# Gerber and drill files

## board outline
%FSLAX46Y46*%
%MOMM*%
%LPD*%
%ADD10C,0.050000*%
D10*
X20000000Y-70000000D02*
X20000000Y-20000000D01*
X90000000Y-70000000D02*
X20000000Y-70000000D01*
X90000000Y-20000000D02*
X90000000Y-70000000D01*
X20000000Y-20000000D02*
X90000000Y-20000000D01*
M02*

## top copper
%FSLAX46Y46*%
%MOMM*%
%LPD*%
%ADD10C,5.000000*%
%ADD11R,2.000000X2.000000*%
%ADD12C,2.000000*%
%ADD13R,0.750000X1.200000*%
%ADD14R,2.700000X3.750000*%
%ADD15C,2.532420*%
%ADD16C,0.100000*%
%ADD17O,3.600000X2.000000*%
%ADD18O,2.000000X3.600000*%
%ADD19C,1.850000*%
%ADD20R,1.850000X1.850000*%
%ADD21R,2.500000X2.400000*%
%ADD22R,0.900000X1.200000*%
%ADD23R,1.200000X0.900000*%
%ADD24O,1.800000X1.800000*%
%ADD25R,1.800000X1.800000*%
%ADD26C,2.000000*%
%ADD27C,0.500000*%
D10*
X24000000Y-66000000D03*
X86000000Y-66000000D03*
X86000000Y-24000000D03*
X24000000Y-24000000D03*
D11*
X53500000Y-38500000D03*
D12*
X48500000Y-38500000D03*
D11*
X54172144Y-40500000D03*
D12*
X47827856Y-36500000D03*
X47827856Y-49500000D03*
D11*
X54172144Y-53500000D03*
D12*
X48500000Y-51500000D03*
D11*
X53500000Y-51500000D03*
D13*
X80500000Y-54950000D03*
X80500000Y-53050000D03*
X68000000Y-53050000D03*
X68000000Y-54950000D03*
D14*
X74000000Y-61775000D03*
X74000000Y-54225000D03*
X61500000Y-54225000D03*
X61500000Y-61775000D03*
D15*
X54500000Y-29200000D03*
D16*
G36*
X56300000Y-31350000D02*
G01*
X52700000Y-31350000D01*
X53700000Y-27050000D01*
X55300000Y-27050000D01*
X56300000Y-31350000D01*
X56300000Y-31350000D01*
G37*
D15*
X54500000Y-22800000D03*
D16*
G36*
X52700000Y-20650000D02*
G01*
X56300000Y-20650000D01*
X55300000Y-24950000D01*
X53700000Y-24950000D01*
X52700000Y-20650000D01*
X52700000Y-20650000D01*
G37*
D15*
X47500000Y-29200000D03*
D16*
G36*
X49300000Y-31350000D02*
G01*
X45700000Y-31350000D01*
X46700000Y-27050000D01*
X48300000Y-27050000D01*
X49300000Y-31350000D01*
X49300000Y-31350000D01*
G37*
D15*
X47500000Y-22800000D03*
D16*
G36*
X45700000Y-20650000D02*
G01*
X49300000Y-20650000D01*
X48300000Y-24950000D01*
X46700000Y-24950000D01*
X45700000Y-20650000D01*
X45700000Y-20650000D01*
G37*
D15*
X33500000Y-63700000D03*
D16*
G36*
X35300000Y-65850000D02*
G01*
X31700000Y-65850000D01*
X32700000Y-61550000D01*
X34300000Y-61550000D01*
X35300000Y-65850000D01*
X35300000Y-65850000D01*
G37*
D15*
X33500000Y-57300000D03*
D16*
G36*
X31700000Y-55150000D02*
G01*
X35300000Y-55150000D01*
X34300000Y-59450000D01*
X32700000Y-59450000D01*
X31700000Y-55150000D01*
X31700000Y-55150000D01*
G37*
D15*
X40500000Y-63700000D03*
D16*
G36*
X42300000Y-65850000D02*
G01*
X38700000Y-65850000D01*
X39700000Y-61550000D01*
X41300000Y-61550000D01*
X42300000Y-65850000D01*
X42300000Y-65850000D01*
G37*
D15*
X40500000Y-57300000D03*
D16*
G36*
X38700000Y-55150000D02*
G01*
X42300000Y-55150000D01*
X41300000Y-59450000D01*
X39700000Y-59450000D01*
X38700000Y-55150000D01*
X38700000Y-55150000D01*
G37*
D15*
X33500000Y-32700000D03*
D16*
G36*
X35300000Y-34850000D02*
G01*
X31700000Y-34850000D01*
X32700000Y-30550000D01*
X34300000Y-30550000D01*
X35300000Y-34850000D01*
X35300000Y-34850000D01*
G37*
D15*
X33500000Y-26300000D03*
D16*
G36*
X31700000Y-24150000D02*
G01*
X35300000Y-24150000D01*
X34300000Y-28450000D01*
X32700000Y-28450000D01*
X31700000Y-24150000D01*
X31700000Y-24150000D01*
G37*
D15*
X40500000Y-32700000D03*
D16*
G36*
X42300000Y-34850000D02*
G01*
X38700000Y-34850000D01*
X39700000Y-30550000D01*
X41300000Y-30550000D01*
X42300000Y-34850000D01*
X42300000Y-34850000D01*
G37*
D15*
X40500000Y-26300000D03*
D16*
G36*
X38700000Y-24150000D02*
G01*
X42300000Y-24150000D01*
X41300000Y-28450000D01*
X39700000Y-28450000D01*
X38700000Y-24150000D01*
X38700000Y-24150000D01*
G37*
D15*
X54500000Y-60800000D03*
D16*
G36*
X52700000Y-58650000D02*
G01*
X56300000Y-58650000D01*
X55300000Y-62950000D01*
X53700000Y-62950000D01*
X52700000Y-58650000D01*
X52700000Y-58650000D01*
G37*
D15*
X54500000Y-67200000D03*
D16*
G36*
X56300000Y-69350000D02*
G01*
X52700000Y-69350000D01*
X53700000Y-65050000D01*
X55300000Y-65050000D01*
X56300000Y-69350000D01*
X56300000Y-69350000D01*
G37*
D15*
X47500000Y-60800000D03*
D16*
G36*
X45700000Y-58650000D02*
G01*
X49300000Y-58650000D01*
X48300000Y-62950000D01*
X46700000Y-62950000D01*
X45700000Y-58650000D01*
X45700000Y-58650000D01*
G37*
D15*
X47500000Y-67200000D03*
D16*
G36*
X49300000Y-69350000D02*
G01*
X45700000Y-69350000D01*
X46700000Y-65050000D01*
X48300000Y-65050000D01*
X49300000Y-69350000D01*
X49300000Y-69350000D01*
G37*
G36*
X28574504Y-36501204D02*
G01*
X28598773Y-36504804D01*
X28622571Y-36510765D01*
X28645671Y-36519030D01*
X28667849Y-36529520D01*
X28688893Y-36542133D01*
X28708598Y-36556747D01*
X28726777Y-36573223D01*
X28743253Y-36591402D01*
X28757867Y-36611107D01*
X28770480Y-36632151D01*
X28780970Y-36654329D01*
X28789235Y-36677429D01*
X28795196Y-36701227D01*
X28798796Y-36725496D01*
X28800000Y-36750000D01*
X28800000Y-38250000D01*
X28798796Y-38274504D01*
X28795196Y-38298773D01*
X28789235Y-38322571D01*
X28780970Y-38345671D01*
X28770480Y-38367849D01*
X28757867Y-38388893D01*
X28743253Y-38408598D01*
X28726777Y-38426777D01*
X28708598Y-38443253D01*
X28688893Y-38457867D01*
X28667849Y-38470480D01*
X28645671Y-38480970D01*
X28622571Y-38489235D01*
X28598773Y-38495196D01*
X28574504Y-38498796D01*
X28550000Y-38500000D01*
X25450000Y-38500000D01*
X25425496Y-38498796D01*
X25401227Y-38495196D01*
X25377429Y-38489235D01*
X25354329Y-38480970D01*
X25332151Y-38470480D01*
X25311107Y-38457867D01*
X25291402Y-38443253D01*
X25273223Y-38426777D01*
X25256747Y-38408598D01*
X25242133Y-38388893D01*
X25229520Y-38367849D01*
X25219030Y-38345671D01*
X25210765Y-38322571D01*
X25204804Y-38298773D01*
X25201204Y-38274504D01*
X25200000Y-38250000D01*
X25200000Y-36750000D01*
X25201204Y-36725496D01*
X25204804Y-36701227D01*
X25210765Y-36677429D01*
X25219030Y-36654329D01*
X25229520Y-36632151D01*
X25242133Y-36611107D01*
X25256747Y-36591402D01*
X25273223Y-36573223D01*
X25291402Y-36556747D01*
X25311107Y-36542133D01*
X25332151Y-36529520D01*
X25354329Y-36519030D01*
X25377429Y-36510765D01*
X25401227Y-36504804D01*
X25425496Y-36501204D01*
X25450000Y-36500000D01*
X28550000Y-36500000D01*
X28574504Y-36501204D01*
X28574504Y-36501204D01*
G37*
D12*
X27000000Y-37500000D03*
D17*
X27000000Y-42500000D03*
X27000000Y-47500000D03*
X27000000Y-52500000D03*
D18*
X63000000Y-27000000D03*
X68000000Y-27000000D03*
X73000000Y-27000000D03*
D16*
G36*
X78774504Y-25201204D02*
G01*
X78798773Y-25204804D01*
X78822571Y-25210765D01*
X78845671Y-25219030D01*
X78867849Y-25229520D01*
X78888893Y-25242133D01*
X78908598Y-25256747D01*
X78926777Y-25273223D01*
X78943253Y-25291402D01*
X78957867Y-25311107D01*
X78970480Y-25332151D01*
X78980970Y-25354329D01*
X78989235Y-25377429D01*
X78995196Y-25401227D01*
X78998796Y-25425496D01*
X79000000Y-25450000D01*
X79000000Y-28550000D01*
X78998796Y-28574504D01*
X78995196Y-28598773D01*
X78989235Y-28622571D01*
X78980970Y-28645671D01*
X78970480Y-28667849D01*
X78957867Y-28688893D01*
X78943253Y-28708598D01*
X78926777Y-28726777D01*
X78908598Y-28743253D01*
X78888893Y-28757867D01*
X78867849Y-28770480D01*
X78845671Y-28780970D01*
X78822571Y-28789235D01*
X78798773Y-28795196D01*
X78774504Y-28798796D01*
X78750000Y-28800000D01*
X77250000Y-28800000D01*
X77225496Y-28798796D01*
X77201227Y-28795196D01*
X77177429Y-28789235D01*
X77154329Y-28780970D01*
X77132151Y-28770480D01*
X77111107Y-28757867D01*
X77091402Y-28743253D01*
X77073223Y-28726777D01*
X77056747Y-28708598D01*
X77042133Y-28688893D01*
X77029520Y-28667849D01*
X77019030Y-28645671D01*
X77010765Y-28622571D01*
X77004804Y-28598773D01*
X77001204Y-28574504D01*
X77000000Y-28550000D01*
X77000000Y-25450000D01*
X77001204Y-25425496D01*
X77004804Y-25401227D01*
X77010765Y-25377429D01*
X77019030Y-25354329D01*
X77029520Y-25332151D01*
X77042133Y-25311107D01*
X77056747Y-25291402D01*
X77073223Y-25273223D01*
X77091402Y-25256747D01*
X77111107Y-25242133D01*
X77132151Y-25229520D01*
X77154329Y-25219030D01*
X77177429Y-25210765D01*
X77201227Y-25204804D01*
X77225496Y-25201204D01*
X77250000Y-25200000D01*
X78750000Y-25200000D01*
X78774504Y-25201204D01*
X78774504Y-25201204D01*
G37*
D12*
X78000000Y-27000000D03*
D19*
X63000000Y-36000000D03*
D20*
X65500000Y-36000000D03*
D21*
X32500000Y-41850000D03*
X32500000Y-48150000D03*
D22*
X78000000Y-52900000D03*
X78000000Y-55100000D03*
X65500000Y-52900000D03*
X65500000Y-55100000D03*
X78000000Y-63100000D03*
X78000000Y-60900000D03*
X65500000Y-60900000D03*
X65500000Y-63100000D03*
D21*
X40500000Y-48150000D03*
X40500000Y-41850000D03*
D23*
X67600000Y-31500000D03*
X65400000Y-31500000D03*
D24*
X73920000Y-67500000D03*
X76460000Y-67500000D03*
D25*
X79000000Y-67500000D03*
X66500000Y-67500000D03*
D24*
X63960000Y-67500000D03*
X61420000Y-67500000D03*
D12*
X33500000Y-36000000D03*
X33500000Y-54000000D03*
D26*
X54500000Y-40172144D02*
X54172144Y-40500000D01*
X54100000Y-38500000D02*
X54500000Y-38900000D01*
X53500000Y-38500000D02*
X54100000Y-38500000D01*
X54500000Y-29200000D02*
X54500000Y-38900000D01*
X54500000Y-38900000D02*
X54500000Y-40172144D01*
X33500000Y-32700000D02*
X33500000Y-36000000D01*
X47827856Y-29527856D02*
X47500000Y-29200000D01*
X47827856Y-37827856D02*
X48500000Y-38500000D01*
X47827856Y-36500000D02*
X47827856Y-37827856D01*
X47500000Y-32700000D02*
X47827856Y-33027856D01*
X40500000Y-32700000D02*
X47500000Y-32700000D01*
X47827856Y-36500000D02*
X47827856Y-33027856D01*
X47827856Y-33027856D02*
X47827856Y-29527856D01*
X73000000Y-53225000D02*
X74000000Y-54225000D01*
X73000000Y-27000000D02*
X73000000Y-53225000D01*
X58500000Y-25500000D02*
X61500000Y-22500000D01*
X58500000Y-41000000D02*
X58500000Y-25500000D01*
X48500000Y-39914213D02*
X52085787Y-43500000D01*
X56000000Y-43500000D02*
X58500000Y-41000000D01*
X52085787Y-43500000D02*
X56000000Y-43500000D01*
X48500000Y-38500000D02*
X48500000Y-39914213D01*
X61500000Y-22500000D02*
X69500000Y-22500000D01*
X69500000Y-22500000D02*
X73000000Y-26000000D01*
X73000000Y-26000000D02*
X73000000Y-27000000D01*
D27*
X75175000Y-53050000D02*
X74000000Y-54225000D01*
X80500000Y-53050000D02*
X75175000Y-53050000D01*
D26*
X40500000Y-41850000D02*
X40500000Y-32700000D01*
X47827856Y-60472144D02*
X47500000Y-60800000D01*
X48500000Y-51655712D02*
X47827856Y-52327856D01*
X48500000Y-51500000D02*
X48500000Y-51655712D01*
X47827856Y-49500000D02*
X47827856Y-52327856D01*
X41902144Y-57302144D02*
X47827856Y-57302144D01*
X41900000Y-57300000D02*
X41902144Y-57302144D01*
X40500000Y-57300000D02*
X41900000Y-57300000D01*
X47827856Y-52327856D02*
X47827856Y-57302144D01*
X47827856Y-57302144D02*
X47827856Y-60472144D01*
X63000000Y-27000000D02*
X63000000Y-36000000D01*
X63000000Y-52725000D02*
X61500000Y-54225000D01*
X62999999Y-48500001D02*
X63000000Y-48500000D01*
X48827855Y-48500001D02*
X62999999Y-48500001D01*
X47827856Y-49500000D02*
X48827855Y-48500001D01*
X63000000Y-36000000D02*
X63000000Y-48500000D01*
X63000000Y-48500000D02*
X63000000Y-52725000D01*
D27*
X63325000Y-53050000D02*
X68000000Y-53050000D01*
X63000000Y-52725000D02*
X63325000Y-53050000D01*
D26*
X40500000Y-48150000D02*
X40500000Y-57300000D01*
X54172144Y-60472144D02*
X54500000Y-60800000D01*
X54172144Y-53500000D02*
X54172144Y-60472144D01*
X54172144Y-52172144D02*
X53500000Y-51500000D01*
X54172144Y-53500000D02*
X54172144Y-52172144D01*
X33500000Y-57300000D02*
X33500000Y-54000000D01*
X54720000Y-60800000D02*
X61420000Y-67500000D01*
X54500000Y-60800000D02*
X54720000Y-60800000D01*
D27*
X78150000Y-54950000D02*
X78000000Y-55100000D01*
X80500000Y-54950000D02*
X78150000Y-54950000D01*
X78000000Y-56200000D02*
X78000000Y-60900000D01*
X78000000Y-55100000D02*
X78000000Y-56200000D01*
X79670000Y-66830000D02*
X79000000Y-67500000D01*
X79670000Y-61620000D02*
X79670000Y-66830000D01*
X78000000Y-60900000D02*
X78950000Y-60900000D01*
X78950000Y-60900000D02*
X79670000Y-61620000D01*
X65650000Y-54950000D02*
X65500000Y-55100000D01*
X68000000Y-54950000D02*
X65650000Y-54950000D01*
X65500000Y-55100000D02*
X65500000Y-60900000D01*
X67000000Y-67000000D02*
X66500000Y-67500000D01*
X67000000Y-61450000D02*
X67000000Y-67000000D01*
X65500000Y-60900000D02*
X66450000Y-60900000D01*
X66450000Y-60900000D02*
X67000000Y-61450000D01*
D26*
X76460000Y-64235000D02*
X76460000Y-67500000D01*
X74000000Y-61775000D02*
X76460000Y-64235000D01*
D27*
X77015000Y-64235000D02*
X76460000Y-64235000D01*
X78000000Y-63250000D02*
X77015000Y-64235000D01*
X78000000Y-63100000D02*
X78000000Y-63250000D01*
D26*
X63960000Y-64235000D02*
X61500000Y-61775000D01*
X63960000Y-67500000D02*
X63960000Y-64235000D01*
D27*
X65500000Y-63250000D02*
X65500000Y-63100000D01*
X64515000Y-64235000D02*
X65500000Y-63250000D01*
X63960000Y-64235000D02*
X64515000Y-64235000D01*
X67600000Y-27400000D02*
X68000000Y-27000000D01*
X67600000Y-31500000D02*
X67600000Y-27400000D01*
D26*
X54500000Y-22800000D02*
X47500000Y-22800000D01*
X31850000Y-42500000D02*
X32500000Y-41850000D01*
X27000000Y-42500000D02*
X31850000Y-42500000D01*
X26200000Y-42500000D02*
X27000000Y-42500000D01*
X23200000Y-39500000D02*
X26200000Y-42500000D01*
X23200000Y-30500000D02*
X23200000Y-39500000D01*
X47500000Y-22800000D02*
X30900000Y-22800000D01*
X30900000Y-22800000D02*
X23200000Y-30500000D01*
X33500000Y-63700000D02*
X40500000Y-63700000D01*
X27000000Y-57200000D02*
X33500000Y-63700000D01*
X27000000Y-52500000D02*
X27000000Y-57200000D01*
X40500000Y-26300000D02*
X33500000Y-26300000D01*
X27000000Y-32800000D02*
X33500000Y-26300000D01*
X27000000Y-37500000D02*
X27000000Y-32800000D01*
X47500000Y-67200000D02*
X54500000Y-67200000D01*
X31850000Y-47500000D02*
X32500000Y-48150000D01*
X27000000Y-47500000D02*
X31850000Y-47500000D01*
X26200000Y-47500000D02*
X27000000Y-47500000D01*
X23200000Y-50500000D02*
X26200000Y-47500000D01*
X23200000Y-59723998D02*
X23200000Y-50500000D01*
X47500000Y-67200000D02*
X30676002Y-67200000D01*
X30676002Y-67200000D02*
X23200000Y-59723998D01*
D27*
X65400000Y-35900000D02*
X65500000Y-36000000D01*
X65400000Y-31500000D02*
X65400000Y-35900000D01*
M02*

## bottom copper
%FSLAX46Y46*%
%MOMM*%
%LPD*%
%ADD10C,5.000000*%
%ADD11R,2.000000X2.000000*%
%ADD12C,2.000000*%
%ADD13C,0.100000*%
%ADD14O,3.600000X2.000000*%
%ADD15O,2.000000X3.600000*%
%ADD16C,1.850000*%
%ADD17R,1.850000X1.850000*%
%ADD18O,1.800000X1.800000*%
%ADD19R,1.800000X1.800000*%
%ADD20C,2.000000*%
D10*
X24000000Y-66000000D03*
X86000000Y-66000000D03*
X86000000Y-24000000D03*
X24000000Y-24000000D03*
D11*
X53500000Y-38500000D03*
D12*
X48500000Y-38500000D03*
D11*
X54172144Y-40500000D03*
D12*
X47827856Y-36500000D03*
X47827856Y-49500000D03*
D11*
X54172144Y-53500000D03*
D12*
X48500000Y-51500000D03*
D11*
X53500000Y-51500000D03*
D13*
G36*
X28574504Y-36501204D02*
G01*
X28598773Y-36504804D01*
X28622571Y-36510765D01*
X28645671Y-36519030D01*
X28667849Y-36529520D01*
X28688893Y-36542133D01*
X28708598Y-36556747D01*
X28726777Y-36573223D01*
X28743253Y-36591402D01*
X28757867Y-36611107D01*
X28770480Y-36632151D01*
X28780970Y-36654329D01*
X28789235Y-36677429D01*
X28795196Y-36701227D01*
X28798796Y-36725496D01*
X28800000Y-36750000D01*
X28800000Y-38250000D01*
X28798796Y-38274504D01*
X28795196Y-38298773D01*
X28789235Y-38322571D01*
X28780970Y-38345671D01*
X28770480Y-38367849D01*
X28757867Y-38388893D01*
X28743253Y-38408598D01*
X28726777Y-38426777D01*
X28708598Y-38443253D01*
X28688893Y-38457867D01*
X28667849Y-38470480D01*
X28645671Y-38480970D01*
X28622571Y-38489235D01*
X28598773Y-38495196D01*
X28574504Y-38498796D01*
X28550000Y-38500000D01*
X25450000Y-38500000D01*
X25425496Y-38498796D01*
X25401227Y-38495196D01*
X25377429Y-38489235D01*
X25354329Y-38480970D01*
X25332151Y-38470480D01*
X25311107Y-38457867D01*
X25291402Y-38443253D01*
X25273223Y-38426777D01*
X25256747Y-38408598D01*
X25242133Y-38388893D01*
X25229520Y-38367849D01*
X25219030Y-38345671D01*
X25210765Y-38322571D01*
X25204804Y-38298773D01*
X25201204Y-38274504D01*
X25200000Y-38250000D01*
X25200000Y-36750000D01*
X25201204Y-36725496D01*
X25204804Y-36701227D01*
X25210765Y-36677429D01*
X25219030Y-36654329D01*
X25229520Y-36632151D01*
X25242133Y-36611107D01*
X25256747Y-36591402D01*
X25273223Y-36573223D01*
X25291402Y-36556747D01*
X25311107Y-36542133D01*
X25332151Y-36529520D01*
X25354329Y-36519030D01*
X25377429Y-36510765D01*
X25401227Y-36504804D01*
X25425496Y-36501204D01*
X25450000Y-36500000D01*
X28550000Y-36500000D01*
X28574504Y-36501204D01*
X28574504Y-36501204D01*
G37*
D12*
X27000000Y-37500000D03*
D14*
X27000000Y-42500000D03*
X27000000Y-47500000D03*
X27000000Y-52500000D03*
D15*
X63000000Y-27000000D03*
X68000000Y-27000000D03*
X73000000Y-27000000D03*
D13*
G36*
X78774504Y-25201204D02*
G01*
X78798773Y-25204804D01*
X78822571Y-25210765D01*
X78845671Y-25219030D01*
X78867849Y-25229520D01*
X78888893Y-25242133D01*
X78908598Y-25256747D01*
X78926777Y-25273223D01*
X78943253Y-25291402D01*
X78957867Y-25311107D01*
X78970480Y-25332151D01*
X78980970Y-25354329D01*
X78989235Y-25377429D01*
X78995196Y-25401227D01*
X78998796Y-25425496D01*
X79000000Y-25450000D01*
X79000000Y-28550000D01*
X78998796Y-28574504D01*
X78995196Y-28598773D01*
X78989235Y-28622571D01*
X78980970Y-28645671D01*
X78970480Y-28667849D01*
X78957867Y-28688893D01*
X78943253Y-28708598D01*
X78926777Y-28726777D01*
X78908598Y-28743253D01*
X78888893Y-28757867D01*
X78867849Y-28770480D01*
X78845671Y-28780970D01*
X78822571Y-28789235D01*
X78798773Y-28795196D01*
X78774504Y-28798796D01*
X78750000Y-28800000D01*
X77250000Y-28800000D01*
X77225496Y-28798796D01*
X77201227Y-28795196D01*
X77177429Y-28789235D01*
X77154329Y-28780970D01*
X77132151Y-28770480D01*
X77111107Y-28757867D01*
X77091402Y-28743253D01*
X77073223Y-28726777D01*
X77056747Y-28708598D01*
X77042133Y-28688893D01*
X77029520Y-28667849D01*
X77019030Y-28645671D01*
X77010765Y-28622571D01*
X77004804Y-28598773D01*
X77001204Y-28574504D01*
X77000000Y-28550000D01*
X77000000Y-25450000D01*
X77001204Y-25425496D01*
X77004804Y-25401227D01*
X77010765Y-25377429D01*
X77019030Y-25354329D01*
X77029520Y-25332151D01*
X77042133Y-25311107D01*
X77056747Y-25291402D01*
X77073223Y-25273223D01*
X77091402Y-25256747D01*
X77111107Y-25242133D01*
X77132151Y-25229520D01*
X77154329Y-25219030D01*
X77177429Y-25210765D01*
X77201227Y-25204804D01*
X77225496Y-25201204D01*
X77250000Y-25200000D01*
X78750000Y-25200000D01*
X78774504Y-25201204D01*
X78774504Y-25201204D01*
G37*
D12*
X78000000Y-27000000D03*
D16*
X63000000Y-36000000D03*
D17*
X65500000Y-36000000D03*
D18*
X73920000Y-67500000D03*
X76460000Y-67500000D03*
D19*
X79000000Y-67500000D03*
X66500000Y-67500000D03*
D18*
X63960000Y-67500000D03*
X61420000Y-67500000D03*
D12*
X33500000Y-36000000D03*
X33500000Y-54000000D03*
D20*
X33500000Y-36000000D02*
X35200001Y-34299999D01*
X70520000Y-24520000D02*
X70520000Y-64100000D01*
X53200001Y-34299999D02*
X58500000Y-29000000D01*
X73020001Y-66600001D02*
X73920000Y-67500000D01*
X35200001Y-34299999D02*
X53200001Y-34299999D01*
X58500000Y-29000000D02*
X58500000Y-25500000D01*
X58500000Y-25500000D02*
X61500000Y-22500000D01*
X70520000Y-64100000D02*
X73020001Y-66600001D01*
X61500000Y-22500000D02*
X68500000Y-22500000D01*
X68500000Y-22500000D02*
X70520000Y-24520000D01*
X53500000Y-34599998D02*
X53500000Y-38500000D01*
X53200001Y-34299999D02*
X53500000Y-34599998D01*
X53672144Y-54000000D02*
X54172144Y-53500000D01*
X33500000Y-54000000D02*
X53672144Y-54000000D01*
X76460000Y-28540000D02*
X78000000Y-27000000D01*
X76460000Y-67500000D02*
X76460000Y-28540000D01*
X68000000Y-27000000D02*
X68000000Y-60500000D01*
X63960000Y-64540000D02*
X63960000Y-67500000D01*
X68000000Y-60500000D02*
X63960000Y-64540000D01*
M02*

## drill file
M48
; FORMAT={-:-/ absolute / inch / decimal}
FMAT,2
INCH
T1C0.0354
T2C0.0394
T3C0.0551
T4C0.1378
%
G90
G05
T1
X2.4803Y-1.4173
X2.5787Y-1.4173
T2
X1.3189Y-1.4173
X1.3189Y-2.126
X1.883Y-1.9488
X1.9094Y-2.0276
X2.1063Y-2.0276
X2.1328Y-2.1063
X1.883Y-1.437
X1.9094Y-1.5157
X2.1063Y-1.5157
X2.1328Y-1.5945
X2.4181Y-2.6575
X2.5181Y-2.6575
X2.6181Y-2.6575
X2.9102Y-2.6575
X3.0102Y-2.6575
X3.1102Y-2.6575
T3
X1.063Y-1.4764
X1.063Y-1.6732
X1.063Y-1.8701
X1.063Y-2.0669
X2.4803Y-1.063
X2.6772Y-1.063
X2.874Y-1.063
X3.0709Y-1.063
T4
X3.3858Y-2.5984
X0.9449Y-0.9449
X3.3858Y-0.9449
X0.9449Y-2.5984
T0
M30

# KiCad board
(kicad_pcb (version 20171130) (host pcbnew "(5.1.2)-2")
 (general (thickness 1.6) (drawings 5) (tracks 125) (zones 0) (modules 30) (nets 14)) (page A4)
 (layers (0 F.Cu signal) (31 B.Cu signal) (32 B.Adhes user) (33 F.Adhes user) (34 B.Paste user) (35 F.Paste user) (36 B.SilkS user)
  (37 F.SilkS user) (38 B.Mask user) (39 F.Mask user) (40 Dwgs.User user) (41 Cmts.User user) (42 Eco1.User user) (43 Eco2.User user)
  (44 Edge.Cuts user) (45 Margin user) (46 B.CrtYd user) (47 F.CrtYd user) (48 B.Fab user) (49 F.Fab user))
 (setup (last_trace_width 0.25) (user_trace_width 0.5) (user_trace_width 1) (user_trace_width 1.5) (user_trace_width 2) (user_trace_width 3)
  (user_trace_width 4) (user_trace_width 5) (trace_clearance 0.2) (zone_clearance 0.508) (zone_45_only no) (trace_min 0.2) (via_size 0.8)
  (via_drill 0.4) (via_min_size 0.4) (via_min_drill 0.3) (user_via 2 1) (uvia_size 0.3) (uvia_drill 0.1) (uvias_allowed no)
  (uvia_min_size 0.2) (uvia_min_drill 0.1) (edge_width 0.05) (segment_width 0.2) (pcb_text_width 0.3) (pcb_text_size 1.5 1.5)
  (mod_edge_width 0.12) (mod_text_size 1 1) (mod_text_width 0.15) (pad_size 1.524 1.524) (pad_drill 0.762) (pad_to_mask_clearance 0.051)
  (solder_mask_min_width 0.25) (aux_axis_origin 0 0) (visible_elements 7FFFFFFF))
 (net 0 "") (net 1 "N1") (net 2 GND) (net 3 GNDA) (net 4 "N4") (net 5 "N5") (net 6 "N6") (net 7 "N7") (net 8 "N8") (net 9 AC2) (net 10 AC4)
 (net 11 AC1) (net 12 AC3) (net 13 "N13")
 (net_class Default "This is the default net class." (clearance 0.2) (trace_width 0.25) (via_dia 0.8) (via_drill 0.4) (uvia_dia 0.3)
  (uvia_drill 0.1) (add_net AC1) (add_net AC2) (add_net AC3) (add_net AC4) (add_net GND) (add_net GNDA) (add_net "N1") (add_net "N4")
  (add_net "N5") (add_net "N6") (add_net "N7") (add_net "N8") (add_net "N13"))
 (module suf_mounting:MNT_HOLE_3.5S (layer F.Cu) (at 24 66)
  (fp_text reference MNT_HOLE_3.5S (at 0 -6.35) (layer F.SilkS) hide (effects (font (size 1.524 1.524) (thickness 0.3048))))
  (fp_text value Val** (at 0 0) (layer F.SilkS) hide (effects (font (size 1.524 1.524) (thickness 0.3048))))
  (pad "" thru_hole circle (at 0 0) (size 5 5) (drill 3.5) (layers *.Cu *.Mask F.SilkS)))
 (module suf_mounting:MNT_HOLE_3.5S (layer F.Cu) (at 86 66)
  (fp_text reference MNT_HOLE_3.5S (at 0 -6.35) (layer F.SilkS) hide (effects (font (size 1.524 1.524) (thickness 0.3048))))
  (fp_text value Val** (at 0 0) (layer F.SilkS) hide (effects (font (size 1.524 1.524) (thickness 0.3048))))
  (pad "" thru_hole circle (at 0 0) (size 5 5) (drill 3.5) (layers *.Cu *.Mask F.SilkS)))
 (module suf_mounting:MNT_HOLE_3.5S (layer F.Cu) (at 86 24)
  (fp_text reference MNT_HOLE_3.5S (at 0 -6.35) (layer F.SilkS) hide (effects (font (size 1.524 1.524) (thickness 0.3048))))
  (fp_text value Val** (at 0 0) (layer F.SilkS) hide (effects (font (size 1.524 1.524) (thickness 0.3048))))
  (pad "" thru_hole circle (at 0 0) (size 5 5) (drill 3.5) (layers *.Cu *.Mask F.SilkS)))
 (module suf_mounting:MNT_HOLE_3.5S (layer F.Cu) (at 24 24)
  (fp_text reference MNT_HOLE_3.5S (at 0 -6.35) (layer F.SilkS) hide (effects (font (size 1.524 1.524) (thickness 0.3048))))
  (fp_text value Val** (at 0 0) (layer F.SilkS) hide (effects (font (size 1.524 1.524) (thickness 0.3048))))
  (pad "" thru_hole circle (at 0 0) (size 5 5) (drill 3.5) (layers *.Cu *.Mask F.SilkS)))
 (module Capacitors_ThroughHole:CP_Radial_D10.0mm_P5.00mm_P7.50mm (layer F.Cu) (at 53.5 38.5 180)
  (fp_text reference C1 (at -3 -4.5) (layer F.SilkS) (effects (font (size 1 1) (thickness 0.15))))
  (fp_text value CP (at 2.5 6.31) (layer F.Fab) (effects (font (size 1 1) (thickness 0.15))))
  (pad 1 thru_hole rect (at 0 0 180) (size 2 2) (drill 1) (layers *.Cu *.Mask) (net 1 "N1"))
  (pad 2 thru_hole circle (at 5 0 180) (size 2 2) (drill 1) (layers *.Cu *.Mask) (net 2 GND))
  (pad 1 thru_hole rect (at -0.672144 -2 180) (size 2 2) (drill 1) (layers *.Cu *.Mask) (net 1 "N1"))
  (pad 2 thru_hole circle (at 5.672144 2 180) (size 2 2) (drill 1) (layers *.Cu *.Mask) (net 2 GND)))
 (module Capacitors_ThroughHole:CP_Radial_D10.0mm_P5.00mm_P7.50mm (layer F.Cu) (at 53.5 51.5 180)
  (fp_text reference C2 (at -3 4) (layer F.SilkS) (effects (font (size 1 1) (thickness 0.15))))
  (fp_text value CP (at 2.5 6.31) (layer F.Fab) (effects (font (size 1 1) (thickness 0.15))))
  (pad 2 thru_hole circle (at 5.672144 2 180) (size 2 2) (drill 1) (layers *.Cu *.Mask) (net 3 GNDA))
  (pad 1 thru_hole rect (at -0.672144 -2 180) (size 2 2) (drill 1) (layers *.Cu *.Mask) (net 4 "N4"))
  (pad 2 thru_hole circle (at 5 0 180) (size 2 2) (drill 1) (layers *.Cu *.Mask) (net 3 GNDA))
  (pad 1 thru_hole rect (at 0 0 180) (size 2 2) (drill 1) (layers *.Cu *.Mask) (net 4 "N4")))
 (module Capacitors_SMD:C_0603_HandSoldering (layer F.Cu) (at 80.5 54 90)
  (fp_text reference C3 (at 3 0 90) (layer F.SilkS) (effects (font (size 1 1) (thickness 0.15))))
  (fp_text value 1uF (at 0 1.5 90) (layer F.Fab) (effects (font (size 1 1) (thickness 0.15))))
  (pad 1 smd rect (at -0.95 0 90) (size 1.2 0.75) (layers F.Cu F.Paste F.Mask) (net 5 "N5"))
  (pad 2 smd rect (at 0.95 0 90) (size 1.2 0.75) (layers F.Cu F.Paste F.Mask) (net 2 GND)))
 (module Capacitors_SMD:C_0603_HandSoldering (layer F.Cu) (at 68 54 90)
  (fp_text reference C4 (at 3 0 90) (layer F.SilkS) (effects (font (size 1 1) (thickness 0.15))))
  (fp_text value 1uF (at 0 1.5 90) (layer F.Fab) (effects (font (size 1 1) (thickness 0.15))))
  (pad 2 smd rect (at 0.95 0 90) (size 1.2 0.75) (layers F.Cu F.Paste F.Mask) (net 3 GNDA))
  (pad 1 smd rect (at -0.95 0 90) (size 1.2 0.75) (layers F.Cu F.Paste F.Mask) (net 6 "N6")))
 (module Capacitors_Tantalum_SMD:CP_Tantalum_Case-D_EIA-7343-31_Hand (layer F.Cu) (at 74 58 90)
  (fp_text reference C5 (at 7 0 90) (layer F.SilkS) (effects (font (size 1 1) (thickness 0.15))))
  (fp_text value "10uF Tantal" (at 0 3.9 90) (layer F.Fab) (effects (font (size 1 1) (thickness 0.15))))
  (pad 1 smd rect (at -3.775 0 90) (size 3.75 2.7) (layers F.Cu F.Paste F.Mask) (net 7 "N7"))
  (pad 2 smd rect (at 3.775 0 90) (size 3.75 2.7) (layers F.Cu F.Paste F.Mask) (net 2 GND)))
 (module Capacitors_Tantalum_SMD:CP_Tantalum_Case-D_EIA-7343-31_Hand (layer F.Cu) (at 61.5 58 90)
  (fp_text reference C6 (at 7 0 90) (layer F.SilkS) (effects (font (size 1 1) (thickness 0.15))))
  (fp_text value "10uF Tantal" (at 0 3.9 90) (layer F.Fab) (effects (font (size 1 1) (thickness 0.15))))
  (pad 2 smd rect (at 3.775 0 90) (size 3.75 2.7) (layers F.Cu F.Paste F.Mask) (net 3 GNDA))
  (pad 1 smd rect (at -3.775 0 90) (size 3.75 2.7) (layers F.Cu F.Paste F.Mask) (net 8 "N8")))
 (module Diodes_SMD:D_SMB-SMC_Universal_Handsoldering (layer F.Cu) (at 54.5 26 90)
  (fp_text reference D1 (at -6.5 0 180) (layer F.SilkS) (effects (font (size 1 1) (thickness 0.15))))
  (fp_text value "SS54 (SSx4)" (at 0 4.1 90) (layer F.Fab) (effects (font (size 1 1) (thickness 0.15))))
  (pad 1 smd trapezoid (at -3.2 0 90) (size 4.3 2.6) (rect_delta 1 0) (layers F.Cu F.Paste F.Mask) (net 1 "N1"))
  (pad 2 smd trapezoid (at 3.2 0 270) (size 4.3 2.6) (rect_delta 1 0) (layers F.Cu F.Paste F.Mask) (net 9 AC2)))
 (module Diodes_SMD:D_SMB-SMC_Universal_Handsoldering (layer F.Cu) (at 47.5 26 270)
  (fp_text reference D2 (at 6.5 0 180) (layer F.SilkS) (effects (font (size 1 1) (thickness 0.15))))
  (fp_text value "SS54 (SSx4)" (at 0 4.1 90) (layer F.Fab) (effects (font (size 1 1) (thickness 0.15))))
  (pad 2 smd trapezoid (at 3.2 0 90) (size 4.3 2.6) (rect_delta 1 0) (layers F.Cu F.Paste F.Mask) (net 2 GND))
  (pad 1 smd trapezoid (at -3.2 0 270) (size 4.3 2.6) (rect_delta 1 0) (layers F.Cu F.Paste F.Mask) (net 9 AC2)))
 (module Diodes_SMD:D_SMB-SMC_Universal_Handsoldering (layer F.Cu) (at 33.5 60.5 270)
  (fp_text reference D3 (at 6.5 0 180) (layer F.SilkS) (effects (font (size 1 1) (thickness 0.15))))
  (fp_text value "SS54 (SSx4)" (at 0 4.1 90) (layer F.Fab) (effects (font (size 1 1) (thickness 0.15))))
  (pad 2 smd trapezoid (at 3.2 0 90) (size 4.3 2.6) (rect_delta 1 0) (layers F.Cu F.Paste F.Mask) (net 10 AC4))
  (pad 1 smd trapezoid (at -3.2 0 270) (size 4.3 2.6) (rect_delta 1 0) (layers F.Cu F.Paste F.Mask) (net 4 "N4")))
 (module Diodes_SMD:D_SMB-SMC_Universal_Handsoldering (layer F.Cu) (at 40.5 60.5 90)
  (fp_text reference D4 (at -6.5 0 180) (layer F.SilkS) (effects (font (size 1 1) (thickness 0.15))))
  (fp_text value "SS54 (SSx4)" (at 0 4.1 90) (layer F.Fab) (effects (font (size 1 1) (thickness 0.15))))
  (pad 1 smd trapezoid (at -3.2 0 90) (size 4.3 2.6) (rect_delta 1 0) (layers F.Cu F.Paste F.Mask) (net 10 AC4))
  (pad 2 smd trapezoid (at 3.2 0 270) (size 4.3 2.6) (rect_delta 1 0) (layers F.Cu F.Paste F.Mask) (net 3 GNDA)))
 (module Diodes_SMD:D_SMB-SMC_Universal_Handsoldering (layer F.Cu) (at 33.5 29.5 90)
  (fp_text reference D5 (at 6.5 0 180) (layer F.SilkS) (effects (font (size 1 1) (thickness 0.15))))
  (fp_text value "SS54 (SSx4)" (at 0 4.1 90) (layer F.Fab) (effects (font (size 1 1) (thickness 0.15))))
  (pad 1 smd trapezoid (at -3.2 0 90) (size 4.3 2.6) (rect_delta 1 0) (layers F.Cu F.Paste F.Mask) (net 1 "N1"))
  (pad 2 smd trapezoid (at 3.2 0 270) (size 4.3 2.6) (rect_delta 1 0) (layers F.Cu F.Paste F.Mask) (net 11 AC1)))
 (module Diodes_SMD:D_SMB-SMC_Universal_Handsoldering (layer F.Cu) (at 40.5 29.5 270)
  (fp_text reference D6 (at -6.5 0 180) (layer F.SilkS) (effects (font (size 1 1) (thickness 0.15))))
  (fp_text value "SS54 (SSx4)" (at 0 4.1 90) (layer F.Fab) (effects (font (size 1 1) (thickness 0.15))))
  (pad 2 smd trapezoid (at 3.2 0 90) (size 4.3 2.6) (rect_delta 1 0) (layers F.Cu F.Paste F.Mask) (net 2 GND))
  (pad 1 smd trapezoid (at -3.2 0 270) (size 4.3 2.6) (rect_delta 1 0) (layers F.Cu F.Paste F.Mask) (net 11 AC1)))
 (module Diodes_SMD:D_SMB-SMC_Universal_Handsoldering (layer F.Cu) (at 54.5 64 270)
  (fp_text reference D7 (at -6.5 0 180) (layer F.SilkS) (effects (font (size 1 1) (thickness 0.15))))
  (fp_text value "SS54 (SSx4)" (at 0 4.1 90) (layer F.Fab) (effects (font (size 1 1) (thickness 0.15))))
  (pad 1 smd trapezoid (at -3.2 0 270) (size 4.3 2.6) (rect_delta 1 0) (layers F.Cu F.Paste F.Mask) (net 4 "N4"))
  (pad 2 smd trapezoid (at 3.2 0 90) (size 4.3 2.6) (rect_delta 1 0) (layers F.Cu F.Paste F.Mask) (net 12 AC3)))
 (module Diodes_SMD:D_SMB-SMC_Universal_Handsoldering (layer F.Cu) (at 47.5 64 90)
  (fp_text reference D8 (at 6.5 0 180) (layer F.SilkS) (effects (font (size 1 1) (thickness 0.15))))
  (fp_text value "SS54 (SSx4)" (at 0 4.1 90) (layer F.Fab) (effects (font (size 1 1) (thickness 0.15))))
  (pad 2 smd trapezoid (at 3.2 0 270) (size 4.3 2.6) (rect_delta 1 0) (layers F.Cu F.Paste F.Mask) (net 3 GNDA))
  (pad 1 smd trapezoid (at -3.2 0 90) (size 4.3 2.6) (rect_delta 1 0) (layers F.Cu F.Paste F.Mask) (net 12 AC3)))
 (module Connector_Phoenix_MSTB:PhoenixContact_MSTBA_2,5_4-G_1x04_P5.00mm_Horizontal (layer F.Cu) (at 27 37.5 270)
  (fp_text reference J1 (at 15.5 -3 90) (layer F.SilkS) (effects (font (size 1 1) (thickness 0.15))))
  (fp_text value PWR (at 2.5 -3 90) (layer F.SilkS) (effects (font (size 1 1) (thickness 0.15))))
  (pad 1 thru_hole roundrect (at 0 0 270) (size 2 3.6) (drill 1.4) (layers *.Cu *.Mask) (roundrect_rratio 0.125) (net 11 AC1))
  (pad 2 thru_hole oval (at 5 0 270) (size 2 3.6) (drill 1.4) (layers *.Cu *.Mask) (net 9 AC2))
  (pad 3 thru_hole oval (at 10 0 270) (size 2 3.6) (drill 1.4) (layers *.Cu *.Mask) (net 12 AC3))
  (pad 4 thru_hole oval (at 15 0 270) (size 2 3.6) (drill 1.4) (layers *.Cu *.Mask) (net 10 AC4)))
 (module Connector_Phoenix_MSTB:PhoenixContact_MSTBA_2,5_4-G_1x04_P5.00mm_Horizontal (layer F.Cu) (at 78 27 180)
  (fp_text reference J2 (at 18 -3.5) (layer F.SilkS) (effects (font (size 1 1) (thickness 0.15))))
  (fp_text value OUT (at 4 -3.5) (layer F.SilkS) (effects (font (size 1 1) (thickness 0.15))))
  (pad 4 thru_hole oval (at 15 0 180) (size 2 3.6) (drill 1.4) (layers *.Cu *.Mask) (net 3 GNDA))
  (pad 3 thru_hole oval (at 10 0 180) (size 2 3.6) (drill 1.4) (layers *.Cu *.Mask) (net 8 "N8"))
  (pad 2 thru_hole oval (at 5 0 180) (size 2 3.6) (drill 1.4) (layers *.Cu *.Mask) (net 2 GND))
  (pad 1 thru_hole roundrect (at 0 0 180) (size 2 3.6) (drill 1.4) (layers *.Cu *.Mask) (roundrect_rratio 0.125) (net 7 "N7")))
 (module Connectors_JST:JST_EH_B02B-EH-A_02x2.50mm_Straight (layer F.Cu) (at 65.5 36 180)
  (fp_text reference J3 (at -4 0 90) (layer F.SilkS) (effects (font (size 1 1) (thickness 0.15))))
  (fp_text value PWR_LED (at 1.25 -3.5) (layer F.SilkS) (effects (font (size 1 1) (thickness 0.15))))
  (pad 2 thru_hole circle (at 2.5 0 180) (size 1.85 1.85) (drill 0.9) (layers *.Cu *.Mask) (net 3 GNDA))
  (pad 1 thru_hole rect (at 0 0 180) (size 1.85 1.85) (drill 0.9) (layers *.Cu *.Mask) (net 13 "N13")))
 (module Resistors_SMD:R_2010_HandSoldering (layer F.Cu) (at 32.5 45 90)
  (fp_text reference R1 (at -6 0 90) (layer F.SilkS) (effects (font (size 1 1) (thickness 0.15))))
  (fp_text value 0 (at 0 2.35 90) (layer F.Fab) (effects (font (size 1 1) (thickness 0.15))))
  (pad 2 smd rect (at 3.15 0 90) (size 2.4 2.5) (layers F.Cu F.Paste F.Mask) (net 9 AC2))
  (pad 1 smd rect (at -3.15 0 90) (size 2.4 2.5) (layers F.Cu F.Paste F.Mask) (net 12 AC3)))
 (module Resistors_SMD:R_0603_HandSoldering (layer F.Cu) (at 78 54 90)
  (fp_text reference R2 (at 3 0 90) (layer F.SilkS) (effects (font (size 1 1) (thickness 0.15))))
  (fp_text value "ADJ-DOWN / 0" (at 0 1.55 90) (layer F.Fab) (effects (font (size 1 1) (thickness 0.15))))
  (pad 2 smd rect (at 1.1 0 90) (size 1.2 0.9) (layers F.Cu F.Paste F.Mask) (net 2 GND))
  (pad 1 smd rect (at -1.1 0 90) (size 1.2 0.9) (layers F.Cu F.Paste F.Mask) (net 5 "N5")))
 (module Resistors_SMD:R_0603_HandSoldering (layer F.Cu) (at 65.5 54 90)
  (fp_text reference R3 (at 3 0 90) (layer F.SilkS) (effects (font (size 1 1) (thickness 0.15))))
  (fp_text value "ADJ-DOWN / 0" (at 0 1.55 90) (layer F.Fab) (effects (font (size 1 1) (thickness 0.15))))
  (pad 2 smd rect (at 1.1 0 90) (size 1.2 0.9) (layers F.Cu F.Paste F.Mask) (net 3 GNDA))
  (pad 1 smd rect (at -1.1 0 90) (size 1.2 0.9) (layers F.Cu F.Paste F.Mask) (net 6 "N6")))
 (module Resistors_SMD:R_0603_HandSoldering (layer F.Cu) (at 78 62 90)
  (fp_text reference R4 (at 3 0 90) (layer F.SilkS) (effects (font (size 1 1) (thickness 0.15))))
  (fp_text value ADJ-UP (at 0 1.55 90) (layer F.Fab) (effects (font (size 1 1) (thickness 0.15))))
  (pad 1 smd rect (at -1.1 0 90) (size 1.2 0.9) (layers F.Cu F.Paste F.Mask) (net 7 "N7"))
  (pad 2 smd rect (at 1.1 0 90) (size 1.2 0.9) (layers F.Cu F.Paste F.Mask) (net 5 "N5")))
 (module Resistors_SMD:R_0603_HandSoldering (layer F.Cu) (at 65.5 62 90)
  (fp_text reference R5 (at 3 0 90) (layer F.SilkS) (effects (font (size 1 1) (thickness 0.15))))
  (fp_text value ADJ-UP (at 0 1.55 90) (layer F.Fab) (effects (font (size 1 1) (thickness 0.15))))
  (pad 2 smd rect (at 1.1 0 90) (size 1.2 0.9) (layers F.Cu F.Paste F.Mask) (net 6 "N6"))
  (pad 1 smd rect (at -1.1 0 90) (size 1.2 0.9) (layers F.Cu F.Paste F.Mask) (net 8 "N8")))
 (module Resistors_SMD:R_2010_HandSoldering (layer F.Cu) (at 40.5 45 90)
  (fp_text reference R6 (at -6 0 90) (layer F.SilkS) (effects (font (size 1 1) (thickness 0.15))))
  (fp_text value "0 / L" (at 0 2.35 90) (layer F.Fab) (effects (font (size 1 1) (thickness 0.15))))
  (pad 1 smd rect (at -3.15 0 90) (size 2.4 2.5) (layers F.Cu F.Paste F.Mask) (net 3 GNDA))
  (pad 2 smd rect (at 3.15 0 90) (size 2.4 2.5) (layers F.Cu F.Paste F.Mask) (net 2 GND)))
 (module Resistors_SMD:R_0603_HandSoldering (layer F.Cu) (at 66.5 31.5 180)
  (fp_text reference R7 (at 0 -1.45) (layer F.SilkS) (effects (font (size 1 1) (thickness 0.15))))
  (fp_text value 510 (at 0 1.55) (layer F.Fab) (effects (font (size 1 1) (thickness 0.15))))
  (pad 1 smd rect (at -1.1 0 180) (size 1.2 0.9) (layers F.Cu F.Paste F.Mask) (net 8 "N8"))
  (pad 2 smd rect (at 1.1 0 180) (size 1.2 0.9) (layers F.Cu F.Paste F.Mask) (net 13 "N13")))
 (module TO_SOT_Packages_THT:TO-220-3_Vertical (layer F.Cu) (at 79 67.5 180)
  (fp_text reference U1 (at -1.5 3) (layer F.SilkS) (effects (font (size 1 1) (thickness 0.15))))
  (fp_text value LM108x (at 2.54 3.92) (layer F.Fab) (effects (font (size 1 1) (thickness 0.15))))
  (pad 3 thru_hole oval (at 5.08 0 180) (size 1.8 1.8) (drill 1) (layers *.Cu *.Mask) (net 1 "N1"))
  (pad 2 thru_hole oval (at 2.54 0 180) (size 1.8 1.8) (drill 1) (layers *.Cu *.Mask) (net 7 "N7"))
  (pad 1 thru_hole rect (at 0 0 180) (size 1.8 1.8) (drill 1) (layers *.Cu *.Mask) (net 5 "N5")))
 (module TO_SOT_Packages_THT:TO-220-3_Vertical (layer F.Cu) (at 66.5 67.5 180)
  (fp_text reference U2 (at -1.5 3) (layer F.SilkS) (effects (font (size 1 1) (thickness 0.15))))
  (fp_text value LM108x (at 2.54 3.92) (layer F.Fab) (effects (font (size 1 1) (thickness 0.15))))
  (pad 1 thru_hole rect (at 0 0 180) (size 1.8 1.8) (drill 1) (layers *.Cu *.Mask) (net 6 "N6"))
  (pad 2 thru_hole oval (at 2.54 0 180) (size 1.8 1.8) (drill 1) (layers *.Cu *.Mask) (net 8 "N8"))
  (pad 3 thru_hole oval (at 5.08 0 180) (size 1.8 1.8) (drill 1) (layers *.Cu *.Mask) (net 4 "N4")))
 (gr_line (start 20 70) (end 20 20) (layer Edge.Cuts) (width 0.05))
 (gr_line (start 90 70) (end 20 70) (layer Edge.Cuts) (width 0.05))
 (gr_line (start 90 20) (end 90 70) (layer Edge.Cuts) (width 0.05))
 (gr_line (start 20 20) (end 90 20) (layer Edge.Cuts) (width 0.05))
 (segment (start 54.5 40.172144) (end 54.172144 40.5) (width 2) (layer F.Cu) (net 1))
 (segment (start 54.1 38.5) (end 54.5 38.9) (width 2) (layer F.Cu) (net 1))
 (segment (start 53.5 38.5) (end 54.1 38.5) (width 2) (layer F.Cu) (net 1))
 (segment (start 54.5 29.2) (end 54.5 38.9) (width 2) (layer F.Cu) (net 1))
 (segment (start 54.5 38.9) (end 54.5 40.172144) (width 2) (layer F.Cu) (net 1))
 (via (at 33.5 36) (size 2) (drill 1) (layers F.Cu B.Cu) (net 1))
 (segment (start 33.5 32.7) (end 33.5 36) (width 2) (layer F.Cu) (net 1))
 (segment (start 33.5 36) (end 35.200001 34.299999) (width 2) (layer B.Cu) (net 1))
 (segment (start 70.52 24.52) (end 70.52 64.1) (width 2) (layer B.Cu) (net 1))
 (segment (start 53.200001 34.299999) (end 58.5 29) (width 2) (layer B.Cu) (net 1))
 (segment (start 73.020001 66.600001) (end 73.92 67.5) (width 2) (layer B.Cu) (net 1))
 (segment (start 35.200001 34.299999) (end 53.200001 34.299999) (width 2) (layer B.Cu) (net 1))
 (segment (start 58.5 29) (end 58.5 25.5) (width 2) (layer B.Cu) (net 1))
 (segment (start 58.5 25.5) (end 61.5 22.5) (width 2) (layer B.Cu) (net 1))
 (segment (start 70.52 64.1) (end 73.020001 66.600001) (width 2) (layer B.Cu) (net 1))
 (segment (start 61.5 22.5) (end 68.5 22.5) (width 2) (layer B.Cu) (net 1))
 (segment (start 68.5 22.5) (end 70.52 24.52) (width 2) (layer B.Cu) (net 1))
 (segment (start 53.5 34.599998) (end 53.5 38.5) (width 2) (layer B.Cu) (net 1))
 (segment (start 53.200001 34.299999) (end 53.5 34.599998) (width 2) (layer B.Cu) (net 1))
 (segment (start 47.827856 29.527856) (end 47.5 29.2) (width 2) (layer F.Cu) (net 2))
 (segment (start 47.827856 37.827856) (end 48.5 38.5) (width 2) (layer F.Cu) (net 2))
 (segment (start 47.827856 36.5) (end 47.827856 37.827856) (width 2) (layer F.Cu) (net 2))
 (segment (start 47.5 32.7) (end 47.827856 33.027856) (width 2) (layer F.Cu) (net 2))
 (segment (start 40.5 32.7) (end 47.5 32.7) (width 2) (layer F.Cu) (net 2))
 (segment (start 47.827856 36.5) (end 47.827856 33.027856) (width 2) (layer F.Cu) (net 2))
 (segment (start 47.827856 33.027856) (end 47.827856 29.527856) (width 2) (layer F.Cu) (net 2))
 (segment (start 73 53.225) (end 74 54.225) (width 2) (layer F.Cu) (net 2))
 (segment (start 73 27) (end 73 53.225) (width 2) (layer F.Cu) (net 2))
 (segment (start 58.5 25.5) (end 61.5 22.5) (width 2) (layer F.Cu) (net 2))
 (segment (start 58.5 41) (end 58.5 25.5) (width 2) (layer F.Cu) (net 2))
 (segment (start 48.5 39.914213) (end 52.085787 43.5) (width 2) (layer F.Cu) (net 2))
 (segment (start 56 43.5) (end 58.5 41) (width 2) (layer F.Cu) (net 2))
 (segment (start 52.085787 43.5) (end 56 43.5) (width 2) (layer F.Cu) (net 2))
 (segment (start 48.5 38.5) (end 48.5 39.914213) (width 2) (layer F.Cu) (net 2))
 (segment (start 61.5 22.5) (end 69.5 22.5) (width 2) (layer F.Cu) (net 2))
 (segment (start 69.5 22.5) (end 73 26) (width 2) (layer F.Cu) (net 2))
 (segment (start 73 26) (end 73 27) (width 2) (layer F.Cu) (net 2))
 (segment (start 75.175 53.05) (end 74 54.225) (width 0.5) (layer F.Cu) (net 2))
 (segment (start 80.5 53.05) (end 75.175 53.05) (width 0.5) (layer F.Cu) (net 2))
 (segment (start 40.5 41.85) (end 40.5 32.7) (width 2) (layer F.Cu) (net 2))
 (segment (start 47.827856 60.472144) (end 47.5 60.8) (width 2) (layer F.Cu) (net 3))
 (segment (start 48.5 51.655712) (end 47.827856 52.327856) (width 2) (layer F.Cu) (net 3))
 (segment (start 48.5 51.5) (end 48.5 51.655712) (width 2) (layer F.Cu) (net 3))
 (segment (start 47.827856 49.5) (end 47.827856 52.327856) (width 2) (layer F.Cu) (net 3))
 (segment (start 41.902144 57.302144) (end 47.827856 57.302144) (width 2) (layer F.Cu) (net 3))
 (segment (start 41.9 57.3) (end 41.902144 57.302144) (width 2) (layer F.Cu) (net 3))
 (segment (start 40.5 57.3) (end 41.9 57.3) (width 2) (layer F.Cu) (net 3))
 (segment (start 47.827856 52.327856) (end 47.827856 57.302144) (width 2) (layer F.Cu) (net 3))
 (segment (start 47.827856 57.302144) (end 47.827856 60.472144) (width 2) (layer F.Cu) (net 3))
 (segment (start 63 27) (end 63 36) (width 2) (layer F.Cu) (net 3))
 (segment (start 63 52.725) (end 61.5 54.225) (width 2) (layer F.Cu) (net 3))
 (segment (start 62.999999 48.500001) (end 63 48.5) (width 2) (layer F.Cu) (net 3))
 (segment (start 48.827855 48.500001) (end 62.999999 48.500001) (width 2) (layer F.Cu) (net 3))
 (segment (start 47.827856 49.5) (end 48.827855 48.500001) (width 2) (layer F.Cu) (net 3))
 (segment (start 63 36) (end 63 48.5) (width 2) (layer F.Cu) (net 3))
 (segment (start 63 48.5) (end 63 52.725) (width 2) (layer F.Cu) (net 3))
 (segment (start 63.325 53.05) (end 68 53.05) (width 0.5) (layer F.Cu) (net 3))
 (segment (start 63 52.725) (end 63.325 53.05) (width 0.5) (layer F.Cu) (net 3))
 (segment (start 40.5 48.15) (end 40.5 57.3) (width 2) (layer F.Cu) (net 3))
 (segment (start 54.172144 60.472144) (end 54.5 60.8) (width 2) (layer F.Cu) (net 4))
 (segment (start 54.172144 53.5) (end 54.172144 60.472144) (width 2) (layer F.Cu) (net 4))
 (segment (start 54.172144 52.172144) (end 53.5 51.5) (width 2) (layer F.Cu) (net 4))
 (segment (start 54.172144 53.5) (end 54.172144 52.172144) (width 2) (layer F.Cu) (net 4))
 (via (at 33.5 54) (size 2) (drill 1) (layers F.Cu B.Cu) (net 4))
 (segment (start 33.5 57.3) (end 33.5 54) (width 2) (layer F.Cu) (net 4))
 (segment (start 53.672144 54) (end 54.172144 53.5) (width 2) (layer B.Cu) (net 4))
 (segment (start 33.5 54) (end 53.672144 54) (width 2) (layer B.Cu) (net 4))
 (segment (start 54.72 60.8) (end 61.42 67.5) (width 2) (layer F.Cu) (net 4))
 (segment (start 54.5 60.8) (end 54.72 60.8) (width 2) (layer F.Cu) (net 4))
 (segment (start 78.15 54.95) (end 78 55.1) (width 0.5) (layer F.Cu) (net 5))
 (segment (start 80.5 54.95) (end 78.15 54.95) (width 0.5) (layer F.Cu) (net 5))
 (segment (start 78 56.2) (end 78 60.9) (width 0.5) (layer F.Cu) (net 5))
 (segment (start 78 55.1) (end 78 56.2) (width 0.5) (layer F.Cu) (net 5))
 (segment (start 79.67 66.83) (end 79 67.5) (width 0.5) (layer F.Cu) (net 5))
 (segment (start 79.67 61.62) (end 79.67 66.83) (width 0.5) (layer F.Cu) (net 5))
 (segment (start 78 60.9) (end 78.95 60.9) (width 0.5) (layer F.Cu) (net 5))
 (segment (start 78.95 60.9) (end 79.67 61.62) (width 0.5) (layer F.Cu) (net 5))
 (segment (start 65.65 54.95) (end 65.5 55.1) (width 0.5) (layer F.Cu) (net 6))
 (segment (start 68 54.95) (end 65.65 54.95) (width 0.5) (layer F.Cu) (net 6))
 (segment (start 65.5 55.1) (end 65.5 60.9) (width 0.5) (layer F.Cu) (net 6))
 (segment (start 67 67) (end 66.5 67.5) (width 0.5) (layer F.Cu) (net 6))
 (segment (start 67 61.45) (end 67 67) (width 0.5) (layer F.Cu) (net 6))
 (segment (start 65.5 60.9) (end 66.45 60.9) (width 0.5) (layer F.Cu) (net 6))
 (segment (start 66.45 60.9) (end 67 61.45) (width 0.5) (layer F.Cu) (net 6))
 (segment (start 76.46 28.54) (end 78 27) (width 2) (layer B.Cu) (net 7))
 (segment (start 76.46 67.5) (end 76.46 28.54) (width 2) (layer B.Cu) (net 7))
 (segment (start 76.46 64.235) (end 76.46 67.5) (width 2) (layer F.Cu) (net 7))
 (segment (start 74 61.775) (end 76.46 64.235) (width 2) (layer F.Cu) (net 7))
 (segment (start 77.015 64.235) (end 76.46 64.235) (width 0.5) (layer F.Cu) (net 7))
 (segment (start 78 63.25) (end 77.015 64.235) (width 0.5) (layer F.Cu) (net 7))
 (segment (start 78 63.1) (end 78 63.25) (width 0.5) (layer F.Cu) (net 7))
 (segment (start 63.96 64.235) (end 61.5 61.775) (width 2) (layer F.Cu) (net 8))
 (segment (start 63.96 67.5) (end 63.96 64.235) (width 2) (layer F.Cu) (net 8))
 (segment (start 65.5 63.25) (end 65.5 63.1) (width 0.5) (layer F.Cu) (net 8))
 (segment (start 64.515 64.235) (end 65.5 63.25) (width 0.5) (layer F.Cu) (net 8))
 (segment (start 63.96 64.235) (end 64.515 64.235) (width 0.5) (layer F.Cu) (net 8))
 (segment (start 68 27) (end 68 60.5) (width 2) (layer B.Cu) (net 8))
 (segment (start 63.96 64.54) (end 63.96 67.5) (width 2) (layer B.Cu) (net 8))
 (segment (start 68 60.5) (end 63.96 64.54) (width 2) (layer B.Cu) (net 8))
 (segment (start 67.6 27.4) (end 68 27) (width 0.5) (layer F.Cu) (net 8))
 (segment (start 67.6 31.5) (end 67.6 27.4) (width 0.5) (layer F.Cu) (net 8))
 (segment (start 54.5 22.8) (end 47.5 22.8) (width 2) (layer F.Cu) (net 9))
 (segment (start 31.85 42.5) (end 32.5 41.85) (width 2) (layer F.Cu) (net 9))
 (segment (start 27 42.5) (end 31.85 42.5) (width 2) (layer F.Cu) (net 9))
 (segment (start 26.2 42.5) (end 27 42.5) (width 2) (layer F.Cu) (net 9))
 (segment (start 23.2 39.5) (end 26.2 42.5) (width 2) (layer F.Cu) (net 9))
 (segment (start 23.2 30.5) (end 23.2 39.5) (width 2) (layer F.Cu) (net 9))
 (segment (start 47.5 22.8) (end 30.9 22.8) (width 2) (layer F.Cu) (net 9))
 (segment (start 30.9 22.8) (end 23.2 30.5) (width 2) (layer F.Cu) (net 9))
 (segment (start 33.5 63.7) (end 40.5 63.7) (width 2) (layer F.Cu) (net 10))
 (segment (start 27 57.2) (end 33.5 63.7) (width 2) (layer F.Cu) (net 10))
 (segment (start 27 52.5) (end 27 57.2) (width 2) (layer F.Cu) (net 10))
 (segment (start 40.5 26.3) (end 33.5 26.3) (width 2) (layer F.Cu) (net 11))
 (segment (start 27 32.8) (end 33.5 26.3) (width 2) (layer F.Cu) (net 11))
 (segment (start 27 37.5) (end 27 32.8) (width 2) (layer F.Cu) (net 11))
 (segment (start 47.5 67.2) (end 54.5 67.2) (width 2) (layer F.Cu) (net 12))
 (segment (start 31.85 47.5) (end 32.5 48.15) (width 2) (layer F.Cu) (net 12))
 (segment (start 27 47.5) (end 31.85 47.5) (width 2) (layer F.Cu) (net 12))
 (segment (start 26.2 47.5) (end 27 47.5) (width 2) (layer F.Cu) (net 12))
 (segment (start 23.2 50.5) (end 26.2 47.5) (width 2) (layer F.Cu) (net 12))
 (segment (start 23.2 59.723998) (end 23.2 50.5) (width 2) (layer F.Cu) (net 12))
 (segment (start 47.5 67.2) (end 30.676002 67.2) (width 2) (layer F.Cu) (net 12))
 (segment (start 30.676002 67.2) (end 23.2 59.723998) (width 2) (layer F.Cu) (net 12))
 (segment (start 65.4 35.9) (end 65.5 36) (width 0.5) (layer F.Cu) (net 13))
 (segment (start 65.4 31.5) (end 65.4 35.9) (width 0.5) (layer F.Cu) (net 13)))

